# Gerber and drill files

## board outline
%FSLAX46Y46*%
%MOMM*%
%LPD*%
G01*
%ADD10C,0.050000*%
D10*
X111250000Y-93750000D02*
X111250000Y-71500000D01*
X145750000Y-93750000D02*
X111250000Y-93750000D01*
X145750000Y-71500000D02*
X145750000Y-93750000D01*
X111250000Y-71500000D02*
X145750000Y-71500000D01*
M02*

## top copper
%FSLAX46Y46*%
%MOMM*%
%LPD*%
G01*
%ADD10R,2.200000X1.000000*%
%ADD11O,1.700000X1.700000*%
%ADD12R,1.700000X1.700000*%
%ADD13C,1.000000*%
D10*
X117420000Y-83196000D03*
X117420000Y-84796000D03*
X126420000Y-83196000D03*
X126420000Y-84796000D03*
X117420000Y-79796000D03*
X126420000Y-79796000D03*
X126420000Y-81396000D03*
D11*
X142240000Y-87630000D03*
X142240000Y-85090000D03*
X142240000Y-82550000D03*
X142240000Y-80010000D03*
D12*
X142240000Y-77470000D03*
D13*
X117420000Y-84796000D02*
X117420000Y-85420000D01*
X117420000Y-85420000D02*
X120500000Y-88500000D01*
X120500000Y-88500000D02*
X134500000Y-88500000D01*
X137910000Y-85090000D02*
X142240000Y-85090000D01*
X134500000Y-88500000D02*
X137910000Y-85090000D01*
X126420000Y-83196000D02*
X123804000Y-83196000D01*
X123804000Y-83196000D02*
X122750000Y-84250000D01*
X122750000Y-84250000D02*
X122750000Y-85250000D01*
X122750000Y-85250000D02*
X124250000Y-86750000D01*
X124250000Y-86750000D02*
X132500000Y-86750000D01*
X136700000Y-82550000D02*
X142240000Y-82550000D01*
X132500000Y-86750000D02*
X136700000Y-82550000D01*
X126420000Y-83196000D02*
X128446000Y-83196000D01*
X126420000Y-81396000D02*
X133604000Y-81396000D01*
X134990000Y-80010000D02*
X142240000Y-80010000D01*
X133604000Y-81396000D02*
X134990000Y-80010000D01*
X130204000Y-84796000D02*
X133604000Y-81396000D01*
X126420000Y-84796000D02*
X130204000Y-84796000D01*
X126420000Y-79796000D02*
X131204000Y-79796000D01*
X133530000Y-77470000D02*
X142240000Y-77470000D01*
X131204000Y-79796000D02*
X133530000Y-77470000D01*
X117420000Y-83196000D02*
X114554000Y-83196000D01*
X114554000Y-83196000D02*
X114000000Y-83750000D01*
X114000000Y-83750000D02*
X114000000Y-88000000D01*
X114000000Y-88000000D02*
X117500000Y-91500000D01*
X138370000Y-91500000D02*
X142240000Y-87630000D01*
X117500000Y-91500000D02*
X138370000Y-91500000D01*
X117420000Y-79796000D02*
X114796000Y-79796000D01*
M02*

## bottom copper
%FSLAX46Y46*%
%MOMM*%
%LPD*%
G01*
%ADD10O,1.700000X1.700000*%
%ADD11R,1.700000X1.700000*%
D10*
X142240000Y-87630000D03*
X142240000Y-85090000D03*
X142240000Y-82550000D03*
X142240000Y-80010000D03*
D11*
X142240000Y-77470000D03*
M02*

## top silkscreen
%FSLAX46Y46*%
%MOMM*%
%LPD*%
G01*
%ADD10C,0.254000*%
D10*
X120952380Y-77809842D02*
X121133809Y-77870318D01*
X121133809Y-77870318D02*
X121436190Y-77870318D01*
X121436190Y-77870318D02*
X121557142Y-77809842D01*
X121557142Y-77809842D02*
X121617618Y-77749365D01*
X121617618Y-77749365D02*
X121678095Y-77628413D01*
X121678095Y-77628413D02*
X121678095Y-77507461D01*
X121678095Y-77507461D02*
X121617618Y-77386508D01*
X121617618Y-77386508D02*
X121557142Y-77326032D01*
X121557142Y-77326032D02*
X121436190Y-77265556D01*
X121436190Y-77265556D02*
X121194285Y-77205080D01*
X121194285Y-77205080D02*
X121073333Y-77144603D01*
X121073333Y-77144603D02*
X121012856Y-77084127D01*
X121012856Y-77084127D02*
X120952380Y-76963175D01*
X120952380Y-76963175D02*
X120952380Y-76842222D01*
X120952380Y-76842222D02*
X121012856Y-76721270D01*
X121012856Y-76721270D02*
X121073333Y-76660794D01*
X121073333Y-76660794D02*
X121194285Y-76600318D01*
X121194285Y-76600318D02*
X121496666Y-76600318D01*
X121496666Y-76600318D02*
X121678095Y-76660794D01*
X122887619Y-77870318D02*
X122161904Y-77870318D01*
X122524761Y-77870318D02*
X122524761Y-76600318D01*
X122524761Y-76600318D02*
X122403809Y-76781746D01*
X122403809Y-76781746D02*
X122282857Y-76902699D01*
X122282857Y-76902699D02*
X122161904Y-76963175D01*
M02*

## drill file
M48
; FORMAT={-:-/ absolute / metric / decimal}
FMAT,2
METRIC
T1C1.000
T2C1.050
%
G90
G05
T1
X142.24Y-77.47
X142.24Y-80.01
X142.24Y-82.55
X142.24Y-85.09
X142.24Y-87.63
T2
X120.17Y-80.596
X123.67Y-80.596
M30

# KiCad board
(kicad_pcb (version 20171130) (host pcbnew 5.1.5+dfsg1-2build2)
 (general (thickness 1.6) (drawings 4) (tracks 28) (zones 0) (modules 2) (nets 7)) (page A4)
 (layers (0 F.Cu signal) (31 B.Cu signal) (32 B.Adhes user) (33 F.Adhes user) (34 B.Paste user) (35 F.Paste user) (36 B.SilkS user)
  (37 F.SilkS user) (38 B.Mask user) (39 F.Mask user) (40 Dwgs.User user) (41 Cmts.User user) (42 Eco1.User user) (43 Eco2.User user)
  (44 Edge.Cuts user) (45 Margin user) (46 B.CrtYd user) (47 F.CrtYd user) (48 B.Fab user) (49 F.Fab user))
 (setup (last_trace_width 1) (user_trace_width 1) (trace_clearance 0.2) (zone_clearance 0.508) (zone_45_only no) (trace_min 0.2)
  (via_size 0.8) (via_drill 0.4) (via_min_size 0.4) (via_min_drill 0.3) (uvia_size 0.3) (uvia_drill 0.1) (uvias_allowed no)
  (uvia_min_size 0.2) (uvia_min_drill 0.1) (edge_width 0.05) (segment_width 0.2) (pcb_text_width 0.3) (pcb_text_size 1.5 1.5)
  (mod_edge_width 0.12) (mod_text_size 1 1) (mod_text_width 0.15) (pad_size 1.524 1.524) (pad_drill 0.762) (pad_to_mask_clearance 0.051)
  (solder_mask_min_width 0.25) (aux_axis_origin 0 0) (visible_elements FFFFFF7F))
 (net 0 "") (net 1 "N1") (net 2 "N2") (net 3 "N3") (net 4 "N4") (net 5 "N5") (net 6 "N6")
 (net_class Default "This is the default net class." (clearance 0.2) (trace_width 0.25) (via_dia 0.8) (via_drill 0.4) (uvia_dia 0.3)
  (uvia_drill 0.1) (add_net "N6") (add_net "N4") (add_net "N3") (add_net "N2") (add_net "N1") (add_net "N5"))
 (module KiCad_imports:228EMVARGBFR (layer F.Cu) (at 121.92 82.296)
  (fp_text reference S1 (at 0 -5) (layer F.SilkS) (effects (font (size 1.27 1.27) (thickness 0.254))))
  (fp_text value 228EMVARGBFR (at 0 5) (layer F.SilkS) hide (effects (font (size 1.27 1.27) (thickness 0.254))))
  (pad MH2 np_thru_hole circle (at 1.75 -1.7) (size 1.05 0) (drill 1.05) (layers *.Cu *.Mask))
  (pad MH1 np_thru_hole circle (at -1.75 -1.7) (size 1.05 0) (drill 1.05) (layers *.Cu *.Mask))
  (pad L4 smd rect (at -4.5 0.9 90) (size 1 2.2) (layers F.Cu F.Paste F.Mask) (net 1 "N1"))
  (pad L3 smd rect (at -4.5 2.5 90) (size 1 2.2) (layers F.Cu F.Paste F.Mask) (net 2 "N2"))
  (pad L2 smd rect (at 4.5 0.9 90) (size 1 2.2) (layers F.Cu F.Paste F.Mask) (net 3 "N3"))
  (pad L1 smd rect (at 4.5 2.5 90) (size 1 2.2) (layers F.Cu F.Paste F.Mask) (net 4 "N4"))
  (pad B2 smd rect (at -4.5 -2.5 90) (size 1 2.2) (layers F.Cu F.Paste F.Mask) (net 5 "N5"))
  (pad B1 smd rect (at 4.5 -2.5 90) (size 1 2.2) (layers F.Cu F.Paste F.Mask) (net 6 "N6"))
  (pad A1 smd rect (at 4.5 -0.9 90) (size 1 2.2) (layers F.Cu F.Paste F.Mask) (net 4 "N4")))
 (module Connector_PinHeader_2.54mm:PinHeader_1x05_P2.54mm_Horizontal (layer B.Cu) (at 142.24 77.47 180)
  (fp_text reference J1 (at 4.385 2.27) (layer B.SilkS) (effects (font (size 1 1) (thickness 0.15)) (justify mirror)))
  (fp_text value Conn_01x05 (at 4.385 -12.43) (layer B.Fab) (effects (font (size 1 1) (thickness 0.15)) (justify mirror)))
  (pad 5 thru_hole oval (at 0 -10.16 180) (size 1.7 1.7) (drill 1) (layers *.Cu *.Mask) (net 1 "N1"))
  (pad 4 thru_hole oval (at 0 -7.62 180) (size 1.7 1.7) (drill 1) (layers *.Cu *.Mask) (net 2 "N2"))
  (pad 3 thru_hole oval (at 0 -5.08 180) (size 1.7 1.7) (drill 1) (layers *.Cu *.Mask) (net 3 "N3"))
  (pad 2 thru_hole oval (at 0 -2.54 180) (size 1.7 1.7) (drill 1) (layers *.Cu *.Mask) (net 4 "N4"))
  (pad 1 thru_hole rect (at 0 0 180) (size 1.7 1.7) (drill 1) (layers *.Cu *.Mask) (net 6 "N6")))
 (gr_line (start 111.25 93.75) (end 111.25 71.5) (layer Edge.Cuts) (width 0.05))
 (gr_line (start 145.75 93.75) (end 111.25 93.75) (layer Edge.Cuts) (width 0.05))
 (gr_line (start 145.75 71.5) (end 145.75 93.75) (layer Edge.Cuts) (width 0.05))
 (gr_line (start 111.25 71.5) (end 145.75 71.5) (layer Edge.Cuts) (width 0.05))
 (segment (start 117.42 84.796) (end 117.42 85.42) (width 1) (layer F.Cu) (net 2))
 (segment (start 117.42 85.42) (end 120.5 88.5) (width 1) (layer F.Cu) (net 2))
 (segment (start 120.5 88.5) (end 134.5 88.5) (width 1) (layer F.Cu) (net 2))
 (segment (start 137.91 85.09) (end 142.24 85.09) (width 1) (layer F.Cu) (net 2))
 (segment (start 134.5 88.5) (end 137.91 85.09) (width 1) (layer F.Cu) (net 2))
 (segment (start 126.42 83.196) (end 123.804 83.196) (width 1) (layer F.Cu) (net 3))
 (segment (start 123.804 83.196) (end 122.75 84.25) (width 1) (layer F.Cu) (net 3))
 (segment (start 122.75 84.25) (end 122.75 85.25) (width 1) (layer F.Cu) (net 3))
 (segment (start 122.75 85.25) (end 124.25 86.75) (width 1) (layer F.Cu) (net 3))
 (segment (start 124.25 86.75) (end 132.5 86.75) (width 1) (layer F.Cu) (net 3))
 (segment (start 136.7 82.55) (end 142.24 82.55) (width 1) (layer F.Cu) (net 3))
 (segment (start 132.5 86.75) (end 136.7 82.55) (width 1) (layer F.Cu) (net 3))
 (segment (start 126.42 83.196) (end 128.446 83.196) (width 1) (layer F.Cu) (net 3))
 (segment (start 126.42 81.396) (end 133.604 81.396) (width 1) (layer F.Cu) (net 4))
 (segment (start 134.99 80.01) (end 142.24 80.01) (width 1) (layer F.Cu) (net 4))
 (segment (start 133.604 81.396) (end 134.99 80.01) (width 1) (layer F.Cu) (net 4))
 (segment (start 130.204 84.796) (end 133.604 81.396) (width 1) (layer F.Cu) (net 4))
 (segment (start 126.42 84.796) (end 130.204 84.796) (width 1) (layer F.Cu) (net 4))
 (segment (start 126.42 79.796) (end 131.204 79.796) (width 1) (layer F.Cu) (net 6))
 (segment (start 133.53 77.47) (end 142.24 77.47) (width 1) (layer F.Cu) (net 6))
 (segment (start 131.204 79.796) (end 133.53 77.47) (width 1) (layer F.Cu) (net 6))
 (segment (start 117.42 83.196) (end 114.554 83.196) (width 1) (layer F.Cu) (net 1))
 (segment (start 114.554 83.196) (end 114 83.75) (width 1) (layer F.Cu) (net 1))
 (segment (start 114 83.75) (end 114 88) (width 1) (layer F.Cu) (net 1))
 (segment (start 114 88) (end 117.5 91.5) (width 1) (layer F.Cu) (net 1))
 (segment (start 138.37 91.5) (end 142.24 87.63) (width 1) (layer F.Cu) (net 1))
 (segment (start 117.5 91.5) (end 138.37 91.5) (width 1) (layer F.Cu) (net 1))
 (segment (start 117.42 79.796) (end 114.796 79.796) (width 1) (layer F.Cu) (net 5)))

